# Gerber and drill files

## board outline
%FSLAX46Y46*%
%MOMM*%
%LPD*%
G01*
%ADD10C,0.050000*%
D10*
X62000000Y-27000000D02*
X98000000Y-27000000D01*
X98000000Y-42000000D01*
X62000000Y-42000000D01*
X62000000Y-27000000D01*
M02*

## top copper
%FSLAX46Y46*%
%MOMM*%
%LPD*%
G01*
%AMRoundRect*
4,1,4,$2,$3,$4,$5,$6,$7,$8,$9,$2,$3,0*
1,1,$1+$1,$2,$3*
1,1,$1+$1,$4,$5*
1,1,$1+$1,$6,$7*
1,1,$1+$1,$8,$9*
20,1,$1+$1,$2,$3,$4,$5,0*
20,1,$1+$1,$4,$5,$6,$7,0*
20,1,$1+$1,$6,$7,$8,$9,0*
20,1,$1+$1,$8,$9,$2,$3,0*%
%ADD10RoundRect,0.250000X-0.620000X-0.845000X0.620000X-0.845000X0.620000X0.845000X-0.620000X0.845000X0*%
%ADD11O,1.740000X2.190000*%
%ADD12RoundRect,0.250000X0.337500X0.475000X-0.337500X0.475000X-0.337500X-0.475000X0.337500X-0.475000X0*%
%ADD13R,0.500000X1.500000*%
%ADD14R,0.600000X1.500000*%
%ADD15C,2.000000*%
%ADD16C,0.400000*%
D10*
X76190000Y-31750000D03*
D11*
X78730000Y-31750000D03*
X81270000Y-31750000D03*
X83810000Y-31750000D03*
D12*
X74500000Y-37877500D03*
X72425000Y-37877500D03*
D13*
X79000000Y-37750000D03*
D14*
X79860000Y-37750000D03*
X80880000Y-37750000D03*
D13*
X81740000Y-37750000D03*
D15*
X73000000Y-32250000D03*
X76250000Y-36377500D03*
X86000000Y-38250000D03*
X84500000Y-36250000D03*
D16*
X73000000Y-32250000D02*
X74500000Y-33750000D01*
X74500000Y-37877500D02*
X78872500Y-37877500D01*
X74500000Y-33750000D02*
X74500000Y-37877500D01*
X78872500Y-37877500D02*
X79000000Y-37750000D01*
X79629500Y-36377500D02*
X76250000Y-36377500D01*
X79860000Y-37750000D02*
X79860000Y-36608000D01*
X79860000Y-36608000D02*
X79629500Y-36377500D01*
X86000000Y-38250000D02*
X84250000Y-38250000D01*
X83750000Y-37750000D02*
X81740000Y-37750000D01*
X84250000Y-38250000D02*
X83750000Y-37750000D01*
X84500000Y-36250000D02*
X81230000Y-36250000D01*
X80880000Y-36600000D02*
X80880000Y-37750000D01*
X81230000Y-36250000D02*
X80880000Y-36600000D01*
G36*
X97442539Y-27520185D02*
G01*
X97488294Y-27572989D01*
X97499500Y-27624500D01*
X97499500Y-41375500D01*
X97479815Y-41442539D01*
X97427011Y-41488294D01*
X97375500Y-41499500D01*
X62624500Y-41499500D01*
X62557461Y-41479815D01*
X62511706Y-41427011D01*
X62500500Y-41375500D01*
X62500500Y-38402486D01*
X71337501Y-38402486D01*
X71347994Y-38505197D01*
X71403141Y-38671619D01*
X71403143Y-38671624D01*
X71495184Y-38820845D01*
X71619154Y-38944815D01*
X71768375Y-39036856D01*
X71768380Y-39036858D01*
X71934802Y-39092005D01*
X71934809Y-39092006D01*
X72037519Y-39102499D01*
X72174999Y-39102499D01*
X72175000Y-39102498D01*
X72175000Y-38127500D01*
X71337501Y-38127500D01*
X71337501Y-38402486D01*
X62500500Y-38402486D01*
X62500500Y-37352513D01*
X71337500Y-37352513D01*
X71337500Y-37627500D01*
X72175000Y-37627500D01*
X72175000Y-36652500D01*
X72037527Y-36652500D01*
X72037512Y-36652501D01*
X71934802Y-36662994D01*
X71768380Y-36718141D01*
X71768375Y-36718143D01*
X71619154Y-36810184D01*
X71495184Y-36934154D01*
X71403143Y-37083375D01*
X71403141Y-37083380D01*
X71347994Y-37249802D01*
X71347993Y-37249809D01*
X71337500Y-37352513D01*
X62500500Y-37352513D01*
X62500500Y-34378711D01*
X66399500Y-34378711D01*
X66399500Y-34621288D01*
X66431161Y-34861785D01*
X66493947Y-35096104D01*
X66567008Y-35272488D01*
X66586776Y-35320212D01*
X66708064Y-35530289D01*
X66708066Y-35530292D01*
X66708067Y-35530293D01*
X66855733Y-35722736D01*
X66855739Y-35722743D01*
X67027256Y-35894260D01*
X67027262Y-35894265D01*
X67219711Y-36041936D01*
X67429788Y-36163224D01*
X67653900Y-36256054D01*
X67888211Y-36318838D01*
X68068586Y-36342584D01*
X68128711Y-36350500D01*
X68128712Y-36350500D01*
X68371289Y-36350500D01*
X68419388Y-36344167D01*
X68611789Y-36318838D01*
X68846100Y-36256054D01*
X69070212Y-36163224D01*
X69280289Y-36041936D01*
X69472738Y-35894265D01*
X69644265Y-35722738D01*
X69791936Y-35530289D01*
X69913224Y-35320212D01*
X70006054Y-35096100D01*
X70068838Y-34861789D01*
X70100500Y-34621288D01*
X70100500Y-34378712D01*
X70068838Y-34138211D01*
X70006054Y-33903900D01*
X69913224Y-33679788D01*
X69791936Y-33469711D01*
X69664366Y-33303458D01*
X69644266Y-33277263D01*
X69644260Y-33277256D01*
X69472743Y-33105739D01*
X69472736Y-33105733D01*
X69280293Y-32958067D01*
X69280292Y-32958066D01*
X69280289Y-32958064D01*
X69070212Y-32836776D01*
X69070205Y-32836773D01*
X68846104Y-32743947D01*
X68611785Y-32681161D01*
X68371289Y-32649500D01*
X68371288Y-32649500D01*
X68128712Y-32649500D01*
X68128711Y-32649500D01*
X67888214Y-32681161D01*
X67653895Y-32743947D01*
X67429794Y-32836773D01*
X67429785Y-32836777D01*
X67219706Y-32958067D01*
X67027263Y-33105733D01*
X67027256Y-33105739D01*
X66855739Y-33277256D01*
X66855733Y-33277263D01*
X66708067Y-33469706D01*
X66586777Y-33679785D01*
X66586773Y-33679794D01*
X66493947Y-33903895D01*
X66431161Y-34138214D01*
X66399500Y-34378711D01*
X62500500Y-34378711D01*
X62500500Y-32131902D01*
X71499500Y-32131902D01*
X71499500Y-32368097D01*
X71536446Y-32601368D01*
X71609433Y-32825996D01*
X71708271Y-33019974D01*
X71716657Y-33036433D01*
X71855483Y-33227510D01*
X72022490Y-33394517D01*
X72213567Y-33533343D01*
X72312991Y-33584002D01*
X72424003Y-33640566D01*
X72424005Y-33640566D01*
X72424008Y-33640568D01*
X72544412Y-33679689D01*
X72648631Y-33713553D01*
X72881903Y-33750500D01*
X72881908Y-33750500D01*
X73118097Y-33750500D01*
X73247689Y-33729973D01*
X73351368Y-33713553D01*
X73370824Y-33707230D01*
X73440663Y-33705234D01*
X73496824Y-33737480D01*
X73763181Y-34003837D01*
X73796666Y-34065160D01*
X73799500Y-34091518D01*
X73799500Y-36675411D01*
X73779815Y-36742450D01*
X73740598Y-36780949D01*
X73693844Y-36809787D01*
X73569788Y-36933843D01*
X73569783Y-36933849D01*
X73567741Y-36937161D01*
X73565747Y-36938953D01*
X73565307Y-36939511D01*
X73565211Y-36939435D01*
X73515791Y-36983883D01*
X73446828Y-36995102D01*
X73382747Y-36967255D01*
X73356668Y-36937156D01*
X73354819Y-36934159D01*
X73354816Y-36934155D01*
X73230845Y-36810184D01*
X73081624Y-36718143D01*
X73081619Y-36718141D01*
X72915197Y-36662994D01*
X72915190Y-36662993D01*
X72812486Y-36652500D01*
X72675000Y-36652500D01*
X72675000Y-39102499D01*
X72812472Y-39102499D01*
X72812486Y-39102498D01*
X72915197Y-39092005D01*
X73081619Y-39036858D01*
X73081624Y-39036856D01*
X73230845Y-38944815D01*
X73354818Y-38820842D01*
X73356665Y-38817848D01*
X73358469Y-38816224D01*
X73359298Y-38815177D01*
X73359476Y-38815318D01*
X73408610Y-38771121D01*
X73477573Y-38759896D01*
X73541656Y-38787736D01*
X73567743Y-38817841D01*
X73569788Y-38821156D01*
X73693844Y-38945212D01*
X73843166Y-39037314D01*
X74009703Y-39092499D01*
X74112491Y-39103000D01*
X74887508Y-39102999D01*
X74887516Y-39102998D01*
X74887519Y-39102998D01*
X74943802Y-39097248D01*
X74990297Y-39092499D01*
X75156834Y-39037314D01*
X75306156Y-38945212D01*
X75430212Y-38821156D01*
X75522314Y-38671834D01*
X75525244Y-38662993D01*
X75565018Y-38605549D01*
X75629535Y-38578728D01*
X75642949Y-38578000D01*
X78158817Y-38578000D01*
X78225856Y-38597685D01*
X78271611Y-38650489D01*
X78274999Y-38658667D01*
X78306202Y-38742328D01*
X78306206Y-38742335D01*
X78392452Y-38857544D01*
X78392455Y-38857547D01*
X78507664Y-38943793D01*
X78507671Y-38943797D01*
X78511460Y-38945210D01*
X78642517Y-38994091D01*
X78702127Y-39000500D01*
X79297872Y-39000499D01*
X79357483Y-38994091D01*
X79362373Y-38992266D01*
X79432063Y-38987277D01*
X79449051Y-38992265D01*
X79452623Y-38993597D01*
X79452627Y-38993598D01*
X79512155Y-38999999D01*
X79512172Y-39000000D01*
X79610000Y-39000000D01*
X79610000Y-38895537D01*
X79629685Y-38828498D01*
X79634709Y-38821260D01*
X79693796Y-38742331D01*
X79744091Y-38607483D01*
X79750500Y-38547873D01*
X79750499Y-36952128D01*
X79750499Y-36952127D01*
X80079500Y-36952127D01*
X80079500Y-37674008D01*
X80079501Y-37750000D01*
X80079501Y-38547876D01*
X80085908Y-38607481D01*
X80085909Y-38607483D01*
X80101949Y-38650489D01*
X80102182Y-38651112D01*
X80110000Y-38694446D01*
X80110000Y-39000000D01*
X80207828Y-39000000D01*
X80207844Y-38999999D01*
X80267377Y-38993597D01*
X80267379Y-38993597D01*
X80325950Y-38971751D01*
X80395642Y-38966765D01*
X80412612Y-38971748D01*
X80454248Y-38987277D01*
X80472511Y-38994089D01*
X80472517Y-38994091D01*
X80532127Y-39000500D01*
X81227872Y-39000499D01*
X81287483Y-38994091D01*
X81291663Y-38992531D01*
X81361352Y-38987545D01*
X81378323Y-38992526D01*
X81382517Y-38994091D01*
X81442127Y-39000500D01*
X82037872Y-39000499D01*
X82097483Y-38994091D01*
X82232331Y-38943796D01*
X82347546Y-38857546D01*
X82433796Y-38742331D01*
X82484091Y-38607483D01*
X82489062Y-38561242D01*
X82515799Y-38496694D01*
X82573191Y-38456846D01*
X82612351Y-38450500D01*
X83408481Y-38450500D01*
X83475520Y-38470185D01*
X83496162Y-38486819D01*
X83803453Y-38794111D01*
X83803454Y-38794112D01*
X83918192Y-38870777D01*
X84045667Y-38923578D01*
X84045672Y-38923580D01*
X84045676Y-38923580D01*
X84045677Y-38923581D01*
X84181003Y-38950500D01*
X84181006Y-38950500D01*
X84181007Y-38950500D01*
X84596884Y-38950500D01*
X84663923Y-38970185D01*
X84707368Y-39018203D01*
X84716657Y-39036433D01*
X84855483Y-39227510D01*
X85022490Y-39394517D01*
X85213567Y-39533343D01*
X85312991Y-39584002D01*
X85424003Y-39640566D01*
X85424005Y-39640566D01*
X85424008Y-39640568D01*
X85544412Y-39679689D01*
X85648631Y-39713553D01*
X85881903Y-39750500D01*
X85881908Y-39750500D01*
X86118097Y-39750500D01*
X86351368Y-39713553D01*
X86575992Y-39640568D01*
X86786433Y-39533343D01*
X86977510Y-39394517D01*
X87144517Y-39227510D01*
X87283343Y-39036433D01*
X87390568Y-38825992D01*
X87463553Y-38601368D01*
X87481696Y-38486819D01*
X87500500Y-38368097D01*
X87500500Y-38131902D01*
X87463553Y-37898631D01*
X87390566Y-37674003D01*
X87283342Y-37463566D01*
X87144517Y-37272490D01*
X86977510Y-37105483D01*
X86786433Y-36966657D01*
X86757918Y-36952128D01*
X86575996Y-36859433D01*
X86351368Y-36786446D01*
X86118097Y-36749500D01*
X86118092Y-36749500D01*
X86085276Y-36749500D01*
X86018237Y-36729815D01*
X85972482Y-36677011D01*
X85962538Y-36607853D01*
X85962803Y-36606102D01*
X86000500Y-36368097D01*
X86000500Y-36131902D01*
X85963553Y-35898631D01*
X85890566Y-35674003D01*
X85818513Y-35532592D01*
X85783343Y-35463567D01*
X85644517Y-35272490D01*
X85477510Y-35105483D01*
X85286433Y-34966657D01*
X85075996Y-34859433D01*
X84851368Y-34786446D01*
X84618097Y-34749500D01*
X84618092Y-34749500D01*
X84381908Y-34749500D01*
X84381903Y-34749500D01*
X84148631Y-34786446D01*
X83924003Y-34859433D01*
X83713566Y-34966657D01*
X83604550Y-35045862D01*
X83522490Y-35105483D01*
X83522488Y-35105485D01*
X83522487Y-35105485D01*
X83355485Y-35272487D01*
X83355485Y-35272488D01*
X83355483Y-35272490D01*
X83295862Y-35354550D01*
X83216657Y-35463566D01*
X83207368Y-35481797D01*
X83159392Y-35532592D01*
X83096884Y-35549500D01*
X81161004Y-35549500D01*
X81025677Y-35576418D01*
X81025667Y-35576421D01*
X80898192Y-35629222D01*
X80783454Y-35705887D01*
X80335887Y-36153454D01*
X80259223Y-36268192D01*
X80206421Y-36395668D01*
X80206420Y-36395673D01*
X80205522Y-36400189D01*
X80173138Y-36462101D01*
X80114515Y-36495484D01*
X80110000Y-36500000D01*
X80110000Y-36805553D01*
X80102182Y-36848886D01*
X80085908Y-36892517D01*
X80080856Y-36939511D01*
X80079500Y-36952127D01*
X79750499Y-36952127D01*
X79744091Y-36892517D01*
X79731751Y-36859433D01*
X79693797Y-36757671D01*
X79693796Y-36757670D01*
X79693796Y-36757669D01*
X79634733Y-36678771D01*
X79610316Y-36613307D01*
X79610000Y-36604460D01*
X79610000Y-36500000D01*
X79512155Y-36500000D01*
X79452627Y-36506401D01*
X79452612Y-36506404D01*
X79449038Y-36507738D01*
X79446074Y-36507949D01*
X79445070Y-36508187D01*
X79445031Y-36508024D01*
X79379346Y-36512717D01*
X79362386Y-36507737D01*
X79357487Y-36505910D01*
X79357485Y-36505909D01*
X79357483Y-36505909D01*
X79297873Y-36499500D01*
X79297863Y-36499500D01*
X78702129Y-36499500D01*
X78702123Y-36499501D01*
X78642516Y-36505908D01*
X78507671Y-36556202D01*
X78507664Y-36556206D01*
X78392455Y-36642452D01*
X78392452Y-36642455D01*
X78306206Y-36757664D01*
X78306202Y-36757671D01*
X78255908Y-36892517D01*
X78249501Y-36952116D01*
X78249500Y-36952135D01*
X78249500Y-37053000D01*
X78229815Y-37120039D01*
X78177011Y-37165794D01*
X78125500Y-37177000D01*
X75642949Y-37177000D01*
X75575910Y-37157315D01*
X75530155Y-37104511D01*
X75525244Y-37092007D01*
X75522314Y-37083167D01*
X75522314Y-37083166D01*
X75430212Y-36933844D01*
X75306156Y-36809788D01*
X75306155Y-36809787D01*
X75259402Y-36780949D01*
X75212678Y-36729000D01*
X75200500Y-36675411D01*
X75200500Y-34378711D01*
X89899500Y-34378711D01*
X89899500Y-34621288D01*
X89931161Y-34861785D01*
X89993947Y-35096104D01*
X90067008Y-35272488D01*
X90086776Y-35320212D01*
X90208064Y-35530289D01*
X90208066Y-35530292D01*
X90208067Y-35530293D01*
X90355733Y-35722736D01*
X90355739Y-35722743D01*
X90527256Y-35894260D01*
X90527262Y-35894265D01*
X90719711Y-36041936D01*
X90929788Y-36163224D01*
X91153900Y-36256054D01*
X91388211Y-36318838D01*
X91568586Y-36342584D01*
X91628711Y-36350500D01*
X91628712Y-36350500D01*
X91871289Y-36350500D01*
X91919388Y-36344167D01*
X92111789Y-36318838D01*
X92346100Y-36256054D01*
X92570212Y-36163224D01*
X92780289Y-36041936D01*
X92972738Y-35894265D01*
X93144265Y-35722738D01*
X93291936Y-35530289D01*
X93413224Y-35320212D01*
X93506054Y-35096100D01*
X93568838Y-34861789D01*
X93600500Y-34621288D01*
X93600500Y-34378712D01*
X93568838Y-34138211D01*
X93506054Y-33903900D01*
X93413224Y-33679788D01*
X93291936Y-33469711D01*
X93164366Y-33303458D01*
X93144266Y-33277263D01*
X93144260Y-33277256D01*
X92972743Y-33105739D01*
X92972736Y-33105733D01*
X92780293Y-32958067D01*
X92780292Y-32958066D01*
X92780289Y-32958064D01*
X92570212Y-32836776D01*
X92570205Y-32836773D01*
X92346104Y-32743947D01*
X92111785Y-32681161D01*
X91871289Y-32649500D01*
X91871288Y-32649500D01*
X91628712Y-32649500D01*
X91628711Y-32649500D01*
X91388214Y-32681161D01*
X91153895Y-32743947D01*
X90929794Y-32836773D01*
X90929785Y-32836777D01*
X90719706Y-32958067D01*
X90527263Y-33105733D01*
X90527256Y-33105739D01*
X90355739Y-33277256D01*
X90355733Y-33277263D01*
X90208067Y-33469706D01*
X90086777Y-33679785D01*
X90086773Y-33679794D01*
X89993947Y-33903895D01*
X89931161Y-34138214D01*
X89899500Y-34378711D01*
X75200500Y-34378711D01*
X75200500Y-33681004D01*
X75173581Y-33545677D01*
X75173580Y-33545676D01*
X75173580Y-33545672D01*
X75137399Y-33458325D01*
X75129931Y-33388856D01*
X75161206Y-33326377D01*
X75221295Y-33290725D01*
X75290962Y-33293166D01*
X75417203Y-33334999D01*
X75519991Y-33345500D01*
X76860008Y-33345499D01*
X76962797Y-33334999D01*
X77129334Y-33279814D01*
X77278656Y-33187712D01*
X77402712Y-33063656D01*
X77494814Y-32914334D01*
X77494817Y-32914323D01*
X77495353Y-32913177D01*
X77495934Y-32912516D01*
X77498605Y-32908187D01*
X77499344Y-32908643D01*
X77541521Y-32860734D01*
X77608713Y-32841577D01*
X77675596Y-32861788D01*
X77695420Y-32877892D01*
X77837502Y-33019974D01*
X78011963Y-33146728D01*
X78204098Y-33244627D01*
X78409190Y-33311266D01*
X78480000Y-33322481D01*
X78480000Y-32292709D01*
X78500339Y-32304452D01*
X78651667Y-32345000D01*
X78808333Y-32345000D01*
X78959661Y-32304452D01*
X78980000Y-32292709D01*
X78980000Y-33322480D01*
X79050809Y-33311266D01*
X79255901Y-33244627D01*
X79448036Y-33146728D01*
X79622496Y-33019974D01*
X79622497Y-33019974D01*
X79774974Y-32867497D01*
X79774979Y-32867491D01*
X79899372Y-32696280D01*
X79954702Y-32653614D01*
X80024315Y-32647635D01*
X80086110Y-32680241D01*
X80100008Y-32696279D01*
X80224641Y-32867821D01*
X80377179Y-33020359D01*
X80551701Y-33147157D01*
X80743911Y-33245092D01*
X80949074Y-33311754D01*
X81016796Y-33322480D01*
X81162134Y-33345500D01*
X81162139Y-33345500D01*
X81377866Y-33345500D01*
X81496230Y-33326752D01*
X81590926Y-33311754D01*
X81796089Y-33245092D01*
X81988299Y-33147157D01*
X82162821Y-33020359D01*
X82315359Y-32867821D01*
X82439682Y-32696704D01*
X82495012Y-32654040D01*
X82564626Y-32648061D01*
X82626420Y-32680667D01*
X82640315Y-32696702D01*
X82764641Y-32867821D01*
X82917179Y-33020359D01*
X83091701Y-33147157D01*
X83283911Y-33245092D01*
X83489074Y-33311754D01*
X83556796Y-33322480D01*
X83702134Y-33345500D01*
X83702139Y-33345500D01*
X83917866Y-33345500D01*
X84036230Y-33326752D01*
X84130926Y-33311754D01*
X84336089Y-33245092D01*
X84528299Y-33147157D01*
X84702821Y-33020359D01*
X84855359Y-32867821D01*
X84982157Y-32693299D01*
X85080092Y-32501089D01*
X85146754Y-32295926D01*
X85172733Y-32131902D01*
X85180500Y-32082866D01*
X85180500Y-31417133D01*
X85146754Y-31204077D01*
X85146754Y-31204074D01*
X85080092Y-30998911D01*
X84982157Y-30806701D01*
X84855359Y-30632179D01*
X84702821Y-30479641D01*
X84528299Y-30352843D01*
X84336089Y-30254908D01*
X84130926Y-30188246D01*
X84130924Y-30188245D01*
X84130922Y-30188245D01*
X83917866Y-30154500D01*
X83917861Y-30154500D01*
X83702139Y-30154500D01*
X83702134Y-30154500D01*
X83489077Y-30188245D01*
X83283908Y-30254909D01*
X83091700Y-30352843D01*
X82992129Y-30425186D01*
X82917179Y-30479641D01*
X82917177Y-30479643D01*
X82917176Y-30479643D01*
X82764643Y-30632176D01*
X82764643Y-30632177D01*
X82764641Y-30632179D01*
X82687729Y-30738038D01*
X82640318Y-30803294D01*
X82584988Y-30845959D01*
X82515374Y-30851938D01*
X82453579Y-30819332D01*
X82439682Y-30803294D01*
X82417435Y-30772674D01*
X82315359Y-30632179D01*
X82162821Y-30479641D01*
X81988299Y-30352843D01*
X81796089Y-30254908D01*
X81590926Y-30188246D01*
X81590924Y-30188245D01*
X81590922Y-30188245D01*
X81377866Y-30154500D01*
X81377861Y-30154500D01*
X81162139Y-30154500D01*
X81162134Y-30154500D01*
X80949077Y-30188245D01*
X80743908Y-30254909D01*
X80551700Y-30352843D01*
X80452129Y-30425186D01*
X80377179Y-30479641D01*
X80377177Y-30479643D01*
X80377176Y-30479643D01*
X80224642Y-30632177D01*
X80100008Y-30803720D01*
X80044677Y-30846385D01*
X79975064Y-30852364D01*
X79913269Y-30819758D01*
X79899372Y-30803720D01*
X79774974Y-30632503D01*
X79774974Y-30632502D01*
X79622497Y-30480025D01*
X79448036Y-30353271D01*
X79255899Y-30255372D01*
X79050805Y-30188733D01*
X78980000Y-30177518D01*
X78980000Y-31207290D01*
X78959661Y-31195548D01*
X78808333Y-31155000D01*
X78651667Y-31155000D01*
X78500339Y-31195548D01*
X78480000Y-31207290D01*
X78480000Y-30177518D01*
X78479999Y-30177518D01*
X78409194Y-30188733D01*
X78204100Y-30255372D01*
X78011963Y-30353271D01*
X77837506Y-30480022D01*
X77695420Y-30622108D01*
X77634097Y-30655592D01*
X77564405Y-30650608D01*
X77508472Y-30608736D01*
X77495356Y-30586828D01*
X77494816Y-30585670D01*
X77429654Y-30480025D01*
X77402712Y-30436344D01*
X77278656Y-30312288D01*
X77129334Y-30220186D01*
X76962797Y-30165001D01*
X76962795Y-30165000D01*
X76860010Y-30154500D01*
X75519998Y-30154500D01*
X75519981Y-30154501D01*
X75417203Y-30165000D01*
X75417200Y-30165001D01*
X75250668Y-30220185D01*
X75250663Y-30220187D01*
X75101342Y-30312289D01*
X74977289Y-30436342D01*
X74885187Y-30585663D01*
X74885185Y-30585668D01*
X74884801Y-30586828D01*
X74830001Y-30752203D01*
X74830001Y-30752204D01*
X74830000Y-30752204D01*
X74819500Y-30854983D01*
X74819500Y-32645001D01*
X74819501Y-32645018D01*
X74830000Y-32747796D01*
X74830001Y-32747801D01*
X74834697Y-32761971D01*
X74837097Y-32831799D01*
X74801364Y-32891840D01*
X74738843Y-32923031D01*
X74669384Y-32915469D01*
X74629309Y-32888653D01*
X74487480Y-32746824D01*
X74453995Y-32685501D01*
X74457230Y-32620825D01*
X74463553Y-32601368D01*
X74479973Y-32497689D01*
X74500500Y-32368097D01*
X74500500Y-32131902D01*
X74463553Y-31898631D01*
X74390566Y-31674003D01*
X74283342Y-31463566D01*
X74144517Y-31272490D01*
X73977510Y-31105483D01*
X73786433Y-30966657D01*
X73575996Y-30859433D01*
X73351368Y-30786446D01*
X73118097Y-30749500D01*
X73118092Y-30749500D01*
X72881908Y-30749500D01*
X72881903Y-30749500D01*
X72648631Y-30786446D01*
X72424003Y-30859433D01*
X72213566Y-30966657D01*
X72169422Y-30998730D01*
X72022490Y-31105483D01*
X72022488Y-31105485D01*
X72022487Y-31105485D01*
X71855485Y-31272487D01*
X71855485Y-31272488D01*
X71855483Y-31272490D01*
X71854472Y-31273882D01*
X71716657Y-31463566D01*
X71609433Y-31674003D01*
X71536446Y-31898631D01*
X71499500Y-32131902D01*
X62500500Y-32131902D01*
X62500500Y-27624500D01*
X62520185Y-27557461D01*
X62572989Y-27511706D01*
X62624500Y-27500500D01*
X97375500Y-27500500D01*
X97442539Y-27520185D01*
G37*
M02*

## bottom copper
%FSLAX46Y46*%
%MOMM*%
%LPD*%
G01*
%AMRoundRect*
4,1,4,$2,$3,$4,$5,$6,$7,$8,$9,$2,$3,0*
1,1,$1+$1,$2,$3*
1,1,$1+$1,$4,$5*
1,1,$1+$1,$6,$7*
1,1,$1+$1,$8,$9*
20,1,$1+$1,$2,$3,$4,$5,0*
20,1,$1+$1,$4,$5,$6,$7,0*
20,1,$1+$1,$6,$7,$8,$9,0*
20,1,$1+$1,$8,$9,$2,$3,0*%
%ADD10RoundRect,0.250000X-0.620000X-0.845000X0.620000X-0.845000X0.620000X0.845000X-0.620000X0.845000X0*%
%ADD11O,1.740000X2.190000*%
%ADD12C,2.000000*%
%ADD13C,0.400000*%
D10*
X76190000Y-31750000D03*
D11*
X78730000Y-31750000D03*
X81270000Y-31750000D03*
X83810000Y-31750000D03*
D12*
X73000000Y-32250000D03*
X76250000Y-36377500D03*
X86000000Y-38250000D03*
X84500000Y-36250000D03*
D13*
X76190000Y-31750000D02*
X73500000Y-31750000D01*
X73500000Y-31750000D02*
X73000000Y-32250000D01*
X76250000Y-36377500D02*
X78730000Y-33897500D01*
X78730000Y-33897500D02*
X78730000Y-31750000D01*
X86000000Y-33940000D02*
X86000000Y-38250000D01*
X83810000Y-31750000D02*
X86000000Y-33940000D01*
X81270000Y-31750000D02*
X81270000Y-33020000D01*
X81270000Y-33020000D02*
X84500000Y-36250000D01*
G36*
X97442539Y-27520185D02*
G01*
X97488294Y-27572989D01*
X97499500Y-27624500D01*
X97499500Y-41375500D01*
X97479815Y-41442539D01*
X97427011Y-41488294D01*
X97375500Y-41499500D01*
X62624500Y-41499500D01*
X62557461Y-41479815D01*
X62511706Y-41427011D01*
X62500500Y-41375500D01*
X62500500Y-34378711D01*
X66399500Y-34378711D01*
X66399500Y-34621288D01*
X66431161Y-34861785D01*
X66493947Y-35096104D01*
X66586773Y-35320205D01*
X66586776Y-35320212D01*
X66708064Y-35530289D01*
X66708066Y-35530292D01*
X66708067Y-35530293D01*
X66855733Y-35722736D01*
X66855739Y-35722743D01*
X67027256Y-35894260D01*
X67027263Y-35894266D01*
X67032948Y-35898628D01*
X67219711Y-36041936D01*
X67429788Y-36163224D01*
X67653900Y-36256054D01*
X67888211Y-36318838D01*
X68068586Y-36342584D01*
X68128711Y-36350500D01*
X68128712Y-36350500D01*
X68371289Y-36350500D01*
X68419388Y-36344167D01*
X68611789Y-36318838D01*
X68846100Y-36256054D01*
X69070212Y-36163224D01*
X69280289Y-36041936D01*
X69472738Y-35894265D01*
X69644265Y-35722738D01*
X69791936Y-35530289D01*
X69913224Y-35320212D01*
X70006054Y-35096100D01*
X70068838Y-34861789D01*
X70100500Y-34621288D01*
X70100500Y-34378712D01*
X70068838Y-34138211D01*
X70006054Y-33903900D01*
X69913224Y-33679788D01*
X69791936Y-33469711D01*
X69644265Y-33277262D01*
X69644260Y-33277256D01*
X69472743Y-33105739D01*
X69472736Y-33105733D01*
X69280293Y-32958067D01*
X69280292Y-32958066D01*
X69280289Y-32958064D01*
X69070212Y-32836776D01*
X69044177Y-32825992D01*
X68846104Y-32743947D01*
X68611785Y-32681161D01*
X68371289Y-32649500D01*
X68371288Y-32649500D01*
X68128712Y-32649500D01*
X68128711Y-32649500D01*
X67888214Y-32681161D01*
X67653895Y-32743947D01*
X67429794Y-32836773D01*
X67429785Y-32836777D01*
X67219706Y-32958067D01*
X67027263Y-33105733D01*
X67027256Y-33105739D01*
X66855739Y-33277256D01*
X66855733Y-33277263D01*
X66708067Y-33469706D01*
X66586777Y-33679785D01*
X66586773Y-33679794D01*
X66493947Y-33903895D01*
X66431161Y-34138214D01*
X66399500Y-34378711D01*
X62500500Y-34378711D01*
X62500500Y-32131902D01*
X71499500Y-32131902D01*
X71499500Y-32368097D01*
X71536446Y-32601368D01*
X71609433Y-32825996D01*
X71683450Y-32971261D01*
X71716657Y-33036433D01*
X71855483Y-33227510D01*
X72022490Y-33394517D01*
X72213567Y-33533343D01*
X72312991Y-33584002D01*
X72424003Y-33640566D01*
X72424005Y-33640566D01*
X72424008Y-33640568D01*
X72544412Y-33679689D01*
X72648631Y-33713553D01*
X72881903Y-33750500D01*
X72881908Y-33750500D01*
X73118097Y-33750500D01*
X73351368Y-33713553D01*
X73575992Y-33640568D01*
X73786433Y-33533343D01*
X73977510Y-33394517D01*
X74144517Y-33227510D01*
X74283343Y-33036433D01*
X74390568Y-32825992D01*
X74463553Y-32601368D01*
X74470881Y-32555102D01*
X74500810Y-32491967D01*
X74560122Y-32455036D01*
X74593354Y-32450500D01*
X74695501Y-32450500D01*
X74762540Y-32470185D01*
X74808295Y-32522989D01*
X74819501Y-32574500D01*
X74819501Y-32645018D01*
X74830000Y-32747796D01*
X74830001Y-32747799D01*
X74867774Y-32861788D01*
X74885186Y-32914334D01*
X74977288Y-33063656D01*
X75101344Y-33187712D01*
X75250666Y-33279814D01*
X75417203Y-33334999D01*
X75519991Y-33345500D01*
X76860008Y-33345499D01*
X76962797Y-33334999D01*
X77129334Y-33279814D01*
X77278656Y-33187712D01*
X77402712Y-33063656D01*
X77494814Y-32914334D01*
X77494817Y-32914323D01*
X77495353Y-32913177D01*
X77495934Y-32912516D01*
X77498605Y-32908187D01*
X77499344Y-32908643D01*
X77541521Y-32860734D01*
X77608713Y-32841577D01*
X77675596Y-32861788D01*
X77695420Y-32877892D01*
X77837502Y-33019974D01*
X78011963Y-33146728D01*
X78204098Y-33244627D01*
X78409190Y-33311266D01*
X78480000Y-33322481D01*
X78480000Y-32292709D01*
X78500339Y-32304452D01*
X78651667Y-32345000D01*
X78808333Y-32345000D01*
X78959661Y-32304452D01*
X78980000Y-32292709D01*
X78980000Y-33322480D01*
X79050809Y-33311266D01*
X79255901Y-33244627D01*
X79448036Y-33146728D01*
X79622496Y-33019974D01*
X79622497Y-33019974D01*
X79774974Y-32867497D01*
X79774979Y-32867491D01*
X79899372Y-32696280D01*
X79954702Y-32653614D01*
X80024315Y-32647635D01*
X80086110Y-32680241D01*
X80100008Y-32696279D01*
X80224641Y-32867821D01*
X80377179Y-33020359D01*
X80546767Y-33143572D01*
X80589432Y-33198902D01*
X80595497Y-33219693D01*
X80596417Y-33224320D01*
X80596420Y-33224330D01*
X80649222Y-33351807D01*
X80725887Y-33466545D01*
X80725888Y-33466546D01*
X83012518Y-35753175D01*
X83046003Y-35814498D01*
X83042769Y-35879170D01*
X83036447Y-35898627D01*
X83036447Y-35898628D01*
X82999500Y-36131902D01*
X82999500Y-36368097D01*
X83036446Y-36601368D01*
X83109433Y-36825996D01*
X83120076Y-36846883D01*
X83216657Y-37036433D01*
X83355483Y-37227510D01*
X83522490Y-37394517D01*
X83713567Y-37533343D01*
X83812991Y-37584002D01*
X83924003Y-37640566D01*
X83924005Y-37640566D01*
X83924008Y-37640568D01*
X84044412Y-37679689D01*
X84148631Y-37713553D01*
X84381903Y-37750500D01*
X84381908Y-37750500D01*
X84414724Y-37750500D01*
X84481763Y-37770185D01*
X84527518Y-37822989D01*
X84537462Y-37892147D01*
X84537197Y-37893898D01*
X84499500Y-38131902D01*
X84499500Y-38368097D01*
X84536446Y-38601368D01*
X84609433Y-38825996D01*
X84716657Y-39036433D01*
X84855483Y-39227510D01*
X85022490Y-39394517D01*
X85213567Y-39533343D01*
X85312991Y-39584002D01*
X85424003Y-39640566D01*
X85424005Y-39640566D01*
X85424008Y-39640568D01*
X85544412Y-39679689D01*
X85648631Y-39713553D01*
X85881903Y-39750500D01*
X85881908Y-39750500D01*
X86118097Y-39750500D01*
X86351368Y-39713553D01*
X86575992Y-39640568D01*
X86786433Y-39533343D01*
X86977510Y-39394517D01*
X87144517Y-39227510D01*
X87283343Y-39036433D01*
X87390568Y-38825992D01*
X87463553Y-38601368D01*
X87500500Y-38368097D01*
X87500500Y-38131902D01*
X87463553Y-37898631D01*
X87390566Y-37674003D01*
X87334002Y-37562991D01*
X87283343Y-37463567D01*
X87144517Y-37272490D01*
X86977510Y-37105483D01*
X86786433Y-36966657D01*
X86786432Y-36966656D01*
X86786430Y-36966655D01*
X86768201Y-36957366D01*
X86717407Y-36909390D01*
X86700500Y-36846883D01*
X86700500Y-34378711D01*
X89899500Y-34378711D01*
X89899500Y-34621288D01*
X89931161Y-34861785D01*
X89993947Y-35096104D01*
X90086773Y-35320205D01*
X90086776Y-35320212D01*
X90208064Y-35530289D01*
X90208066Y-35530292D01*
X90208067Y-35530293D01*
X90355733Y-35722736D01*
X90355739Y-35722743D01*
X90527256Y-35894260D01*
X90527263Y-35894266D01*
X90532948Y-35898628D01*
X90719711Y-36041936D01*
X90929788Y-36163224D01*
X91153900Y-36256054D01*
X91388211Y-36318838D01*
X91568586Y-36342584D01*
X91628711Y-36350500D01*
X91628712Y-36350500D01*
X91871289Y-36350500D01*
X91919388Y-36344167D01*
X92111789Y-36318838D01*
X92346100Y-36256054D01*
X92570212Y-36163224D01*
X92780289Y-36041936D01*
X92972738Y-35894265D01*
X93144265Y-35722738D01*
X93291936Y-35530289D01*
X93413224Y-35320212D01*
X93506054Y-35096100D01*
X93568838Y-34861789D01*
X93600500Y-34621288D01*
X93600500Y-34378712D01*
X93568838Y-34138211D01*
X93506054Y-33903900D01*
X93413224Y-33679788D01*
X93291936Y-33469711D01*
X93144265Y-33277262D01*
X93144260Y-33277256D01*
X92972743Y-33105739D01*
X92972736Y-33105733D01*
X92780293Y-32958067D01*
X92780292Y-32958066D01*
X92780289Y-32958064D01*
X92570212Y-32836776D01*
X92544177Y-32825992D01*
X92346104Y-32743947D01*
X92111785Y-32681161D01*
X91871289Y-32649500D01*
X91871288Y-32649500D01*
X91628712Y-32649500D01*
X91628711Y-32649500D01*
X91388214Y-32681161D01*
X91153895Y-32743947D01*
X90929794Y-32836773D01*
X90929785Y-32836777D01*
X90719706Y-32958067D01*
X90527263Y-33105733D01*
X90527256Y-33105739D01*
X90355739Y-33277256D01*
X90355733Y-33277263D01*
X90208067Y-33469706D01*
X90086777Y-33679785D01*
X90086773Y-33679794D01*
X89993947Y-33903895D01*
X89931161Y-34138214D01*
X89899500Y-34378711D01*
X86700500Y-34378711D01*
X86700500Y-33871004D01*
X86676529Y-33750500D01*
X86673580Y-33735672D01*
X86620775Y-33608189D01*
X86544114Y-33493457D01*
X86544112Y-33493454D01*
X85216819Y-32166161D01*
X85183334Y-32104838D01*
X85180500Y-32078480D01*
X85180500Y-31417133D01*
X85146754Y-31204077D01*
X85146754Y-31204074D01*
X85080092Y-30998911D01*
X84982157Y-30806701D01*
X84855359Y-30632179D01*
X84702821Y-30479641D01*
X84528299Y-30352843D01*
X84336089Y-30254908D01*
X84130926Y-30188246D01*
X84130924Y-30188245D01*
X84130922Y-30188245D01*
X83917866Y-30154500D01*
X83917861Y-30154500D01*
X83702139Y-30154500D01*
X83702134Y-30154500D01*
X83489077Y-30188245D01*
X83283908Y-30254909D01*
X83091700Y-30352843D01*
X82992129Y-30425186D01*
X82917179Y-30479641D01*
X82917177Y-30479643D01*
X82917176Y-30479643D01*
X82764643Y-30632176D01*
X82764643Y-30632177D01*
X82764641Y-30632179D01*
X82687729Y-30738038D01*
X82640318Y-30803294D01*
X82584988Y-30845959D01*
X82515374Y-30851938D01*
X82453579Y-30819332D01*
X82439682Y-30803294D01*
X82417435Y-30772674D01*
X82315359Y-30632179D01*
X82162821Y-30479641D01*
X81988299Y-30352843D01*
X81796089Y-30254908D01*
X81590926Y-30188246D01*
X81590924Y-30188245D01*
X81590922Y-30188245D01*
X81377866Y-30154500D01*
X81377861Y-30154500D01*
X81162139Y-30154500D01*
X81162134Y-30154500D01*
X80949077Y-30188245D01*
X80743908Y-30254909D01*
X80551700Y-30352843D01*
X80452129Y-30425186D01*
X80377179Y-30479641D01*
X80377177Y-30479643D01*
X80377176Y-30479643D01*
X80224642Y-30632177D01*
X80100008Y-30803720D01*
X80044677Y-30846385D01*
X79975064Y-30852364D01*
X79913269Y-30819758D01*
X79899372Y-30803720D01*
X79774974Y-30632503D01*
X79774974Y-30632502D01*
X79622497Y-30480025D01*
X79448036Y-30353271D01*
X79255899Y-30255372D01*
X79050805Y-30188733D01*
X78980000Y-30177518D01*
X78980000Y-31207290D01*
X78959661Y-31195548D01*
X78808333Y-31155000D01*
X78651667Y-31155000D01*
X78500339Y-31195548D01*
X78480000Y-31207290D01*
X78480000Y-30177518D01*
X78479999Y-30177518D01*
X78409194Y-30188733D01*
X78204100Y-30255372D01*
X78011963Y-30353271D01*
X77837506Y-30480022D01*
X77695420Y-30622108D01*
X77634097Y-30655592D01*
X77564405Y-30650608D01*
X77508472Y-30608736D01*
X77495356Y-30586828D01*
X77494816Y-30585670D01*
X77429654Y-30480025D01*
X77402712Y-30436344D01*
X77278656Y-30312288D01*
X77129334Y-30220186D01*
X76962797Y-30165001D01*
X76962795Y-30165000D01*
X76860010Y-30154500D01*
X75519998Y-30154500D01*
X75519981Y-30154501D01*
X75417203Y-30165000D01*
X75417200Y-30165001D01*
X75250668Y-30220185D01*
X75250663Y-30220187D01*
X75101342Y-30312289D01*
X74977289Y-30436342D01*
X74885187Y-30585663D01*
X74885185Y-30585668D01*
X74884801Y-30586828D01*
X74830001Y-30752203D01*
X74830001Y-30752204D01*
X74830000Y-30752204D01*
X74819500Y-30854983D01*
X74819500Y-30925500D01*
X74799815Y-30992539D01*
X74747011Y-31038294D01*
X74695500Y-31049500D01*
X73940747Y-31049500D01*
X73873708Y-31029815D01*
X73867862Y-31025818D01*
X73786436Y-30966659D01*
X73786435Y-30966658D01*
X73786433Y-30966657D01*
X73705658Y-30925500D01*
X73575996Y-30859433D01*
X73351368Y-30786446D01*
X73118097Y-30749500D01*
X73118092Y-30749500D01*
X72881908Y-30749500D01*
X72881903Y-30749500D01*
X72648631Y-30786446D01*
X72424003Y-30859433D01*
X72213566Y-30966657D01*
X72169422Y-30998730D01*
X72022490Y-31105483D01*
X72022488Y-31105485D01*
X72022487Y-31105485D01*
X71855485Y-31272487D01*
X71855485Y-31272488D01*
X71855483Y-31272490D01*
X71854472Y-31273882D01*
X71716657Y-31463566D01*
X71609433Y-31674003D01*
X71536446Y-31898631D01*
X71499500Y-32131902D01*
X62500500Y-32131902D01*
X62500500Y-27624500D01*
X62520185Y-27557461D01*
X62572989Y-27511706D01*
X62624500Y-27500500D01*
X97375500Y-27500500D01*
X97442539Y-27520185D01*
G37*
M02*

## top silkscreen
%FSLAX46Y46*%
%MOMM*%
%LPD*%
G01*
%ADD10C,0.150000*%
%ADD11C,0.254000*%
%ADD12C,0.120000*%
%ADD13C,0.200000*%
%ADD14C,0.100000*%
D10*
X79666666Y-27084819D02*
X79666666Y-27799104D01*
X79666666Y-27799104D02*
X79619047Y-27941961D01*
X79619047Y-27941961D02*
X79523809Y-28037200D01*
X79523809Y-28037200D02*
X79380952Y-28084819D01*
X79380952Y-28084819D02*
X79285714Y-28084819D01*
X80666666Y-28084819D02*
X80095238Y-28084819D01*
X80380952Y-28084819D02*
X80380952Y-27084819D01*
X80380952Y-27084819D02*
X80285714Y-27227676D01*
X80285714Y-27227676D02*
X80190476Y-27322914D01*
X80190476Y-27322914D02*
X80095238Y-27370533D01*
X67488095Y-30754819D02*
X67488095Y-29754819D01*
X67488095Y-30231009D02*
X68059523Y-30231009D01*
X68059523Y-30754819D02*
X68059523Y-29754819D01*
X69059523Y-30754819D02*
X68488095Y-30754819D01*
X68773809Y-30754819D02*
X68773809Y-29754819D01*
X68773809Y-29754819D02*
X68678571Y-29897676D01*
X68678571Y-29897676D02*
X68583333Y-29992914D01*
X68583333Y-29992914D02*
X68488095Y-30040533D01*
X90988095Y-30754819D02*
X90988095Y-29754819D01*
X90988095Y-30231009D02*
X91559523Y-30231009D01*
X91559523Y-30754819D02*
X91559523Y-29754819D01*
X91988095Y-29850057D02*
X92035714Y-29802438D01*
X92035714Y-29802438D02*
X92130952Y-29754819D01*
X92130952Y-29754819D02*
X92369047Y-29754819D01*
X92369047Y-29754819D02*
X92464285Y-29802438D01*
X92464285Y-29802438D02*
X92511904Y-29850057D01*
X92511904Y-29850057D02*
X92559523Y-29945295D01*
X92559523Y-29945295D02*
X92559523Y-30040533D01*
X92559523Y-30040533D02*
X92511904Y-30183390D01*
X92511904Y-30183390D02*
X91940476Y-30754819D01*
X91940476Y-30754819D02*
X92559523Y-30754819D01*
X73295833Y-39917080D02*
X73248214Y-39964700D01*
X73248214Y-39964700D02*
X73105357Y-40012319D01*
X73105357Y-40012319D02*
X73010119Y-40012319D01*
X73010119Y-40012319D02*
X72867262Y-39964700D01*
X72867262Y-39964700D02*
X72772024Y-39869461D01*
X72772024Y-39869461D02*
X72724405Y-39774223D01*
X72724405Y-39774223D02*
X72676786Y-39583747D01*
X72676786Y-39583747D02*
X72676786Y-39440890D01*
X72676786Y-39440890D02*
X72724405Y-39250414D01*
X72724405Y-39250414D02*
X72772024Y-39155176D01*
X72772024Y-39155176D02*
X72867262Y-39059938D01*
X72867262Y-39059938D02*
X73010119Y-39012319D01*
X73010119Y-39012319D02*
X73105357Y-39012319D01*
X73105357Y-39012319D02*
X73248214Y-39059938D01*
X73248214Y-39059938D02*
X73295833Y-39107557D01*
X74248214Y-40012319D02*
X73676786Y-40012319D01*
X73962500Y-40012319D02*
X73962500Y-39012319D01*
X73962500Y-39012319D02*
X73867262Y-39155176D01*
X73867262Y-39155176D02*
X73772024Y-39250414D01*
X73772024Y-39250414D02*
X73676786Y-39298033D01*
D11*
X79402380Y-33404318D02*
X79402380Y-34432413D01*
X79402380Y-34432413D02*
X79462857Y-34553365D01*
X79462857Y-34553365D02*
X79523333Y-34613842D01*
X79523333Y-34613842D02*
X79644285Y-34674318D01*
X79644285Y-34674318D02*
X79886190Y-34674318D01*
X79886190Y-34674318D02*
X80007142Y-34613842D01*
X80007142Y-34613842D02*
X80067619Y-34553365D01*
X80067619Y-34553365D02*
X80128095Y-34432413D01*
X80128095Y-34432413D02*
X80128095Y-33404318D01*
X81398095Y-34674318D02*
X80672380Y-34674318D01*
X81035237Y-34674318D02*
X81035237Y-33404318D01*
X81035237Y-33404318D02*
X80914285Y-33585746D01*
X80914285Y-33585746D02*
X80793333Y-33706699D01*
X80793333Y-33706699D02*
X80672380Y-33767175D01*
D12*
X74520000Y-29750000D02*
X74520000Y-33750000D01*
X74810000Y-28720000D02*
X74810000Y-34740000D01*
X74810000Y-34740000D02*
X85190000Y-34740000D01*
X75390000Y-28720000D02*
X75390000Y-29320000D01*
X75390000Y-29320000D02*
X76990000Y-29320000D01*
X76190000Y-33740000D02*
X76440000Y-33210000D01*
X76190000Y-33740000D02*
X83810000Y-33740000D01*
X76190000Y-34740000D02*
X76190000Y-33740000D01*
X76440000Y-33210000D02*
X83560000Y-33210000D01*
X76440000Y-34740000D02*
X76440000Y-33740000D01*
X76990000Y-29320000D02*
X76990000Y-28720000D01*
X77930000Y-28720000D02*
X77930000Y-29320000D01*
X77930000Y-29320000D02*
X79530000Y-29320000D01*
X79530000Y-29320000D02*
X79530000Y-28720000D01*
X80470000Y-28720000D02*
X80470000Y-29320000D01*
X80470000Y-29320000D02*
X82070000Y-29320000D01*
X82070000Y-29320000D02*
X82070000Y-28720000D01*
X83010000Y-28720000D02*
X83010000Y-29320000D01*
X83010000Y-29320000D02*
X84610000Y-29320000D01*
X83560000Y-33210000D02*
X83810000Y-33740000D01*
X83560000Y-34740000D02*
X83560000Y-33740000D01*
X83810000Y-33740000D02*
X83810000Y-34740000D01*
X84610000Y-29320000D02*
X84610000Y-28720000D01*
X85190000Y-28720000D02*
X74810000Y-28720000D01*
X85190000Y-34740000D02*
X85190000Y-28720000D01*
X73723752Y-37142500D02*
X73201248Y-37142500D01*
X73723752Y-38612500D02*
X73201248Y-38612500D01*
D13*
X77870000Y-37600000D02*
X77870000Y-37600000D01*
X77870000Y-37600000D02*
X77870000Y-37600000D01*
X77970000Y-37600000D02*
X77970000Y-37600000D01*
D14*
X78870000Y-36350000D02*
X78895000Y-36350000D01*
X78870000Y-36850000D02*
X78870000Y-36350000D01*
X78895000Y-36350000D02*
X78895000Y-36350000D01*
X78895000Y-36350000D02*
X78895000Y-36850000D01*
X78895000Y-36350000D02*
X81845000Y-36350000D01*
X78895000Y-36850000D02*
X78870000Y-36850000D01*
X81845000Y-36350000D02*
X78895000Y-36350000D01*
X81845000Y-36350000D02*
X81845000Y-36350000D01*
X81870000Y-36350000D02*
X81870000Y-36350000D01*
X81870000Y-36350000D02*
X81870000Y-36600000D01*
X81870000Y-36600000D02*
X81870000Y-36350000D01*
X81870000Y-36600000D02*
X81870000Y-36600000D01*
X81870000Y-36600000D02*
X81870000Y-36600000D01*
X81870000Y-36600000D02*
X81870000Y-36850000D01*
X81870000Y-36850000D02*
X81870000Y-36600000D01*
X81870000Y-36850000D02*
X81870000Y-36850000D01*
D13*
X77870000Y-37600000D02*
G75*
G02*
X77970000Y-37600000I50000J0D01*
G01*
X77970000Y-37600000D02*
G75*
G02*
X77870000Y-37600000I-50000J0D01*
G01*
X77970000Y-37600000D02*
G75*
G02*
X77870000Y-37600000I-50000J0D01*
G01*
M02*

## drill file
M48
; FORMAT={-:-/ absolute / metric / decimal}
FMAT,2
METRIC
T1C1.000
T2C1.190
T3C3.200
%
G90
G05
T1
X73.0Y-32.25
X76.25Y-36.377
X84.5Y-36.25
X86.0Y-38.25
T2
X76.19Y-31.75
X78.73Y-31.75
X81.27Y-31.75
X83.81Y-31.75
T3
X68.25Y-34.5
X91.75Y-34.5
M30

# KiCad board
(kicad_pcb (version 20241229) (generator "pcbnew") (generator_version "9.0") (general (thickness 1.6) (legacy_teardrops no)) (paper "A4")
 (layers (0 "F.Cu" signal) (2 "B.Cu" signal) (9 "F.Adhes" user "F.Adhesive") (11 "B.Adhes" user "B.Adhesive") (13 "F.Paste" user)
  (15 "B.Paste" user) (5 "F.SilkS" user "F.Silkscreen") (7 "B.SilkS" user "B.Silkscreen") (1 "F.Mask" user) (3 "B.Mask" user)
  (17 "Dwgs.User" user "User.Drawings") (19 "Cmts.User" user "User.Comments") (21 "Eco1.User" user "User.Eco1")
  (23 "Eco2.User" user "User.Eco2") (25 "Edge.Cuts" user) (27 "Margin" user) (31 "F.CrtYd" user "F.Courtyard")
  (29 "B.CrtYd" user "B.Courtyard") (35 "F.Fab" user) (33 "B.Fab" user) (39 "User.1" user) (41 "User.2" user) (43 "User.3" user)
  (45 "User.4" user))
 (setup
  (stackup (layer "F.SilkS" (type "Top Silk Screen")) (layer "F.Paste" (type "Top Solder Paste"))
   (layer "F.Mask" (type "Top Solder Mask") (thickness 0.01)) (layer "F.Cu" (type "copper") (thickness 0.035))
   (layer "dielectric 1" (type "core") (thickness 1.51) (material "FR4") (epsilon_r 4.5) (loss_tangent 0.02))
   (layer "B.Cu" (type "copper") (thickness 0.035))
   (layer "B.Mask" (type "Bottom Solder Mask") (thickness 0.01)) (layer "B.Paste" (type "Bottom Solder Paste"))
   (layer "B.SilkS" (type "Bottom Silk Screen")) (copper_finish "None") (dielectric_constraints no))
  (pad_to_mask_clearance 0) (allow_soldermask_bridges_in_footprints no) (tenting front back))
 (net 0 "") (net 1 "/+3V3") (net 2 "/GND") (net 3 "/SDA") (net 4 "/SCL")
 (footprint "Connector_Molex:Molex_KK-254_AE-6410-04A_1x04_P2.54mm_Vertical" (layer "F.Cu") (at 76.19 31.75)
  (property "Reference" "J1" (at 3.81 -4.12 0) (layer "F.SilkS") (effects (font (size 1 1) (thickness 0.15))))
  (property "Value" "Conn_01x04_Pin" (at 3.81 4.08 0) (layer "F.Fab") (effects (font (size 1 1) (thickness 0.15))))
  (fp_line (start -1.67 -2) (end -1.67 2) (stroke (width 0.12) (type solid)) (layer "F.SilkS"))
  (fp_line (start -1.38 -3.03) (end -1.38 2.99) (stroke (width 0.12) (type solid)) (layer "F.SilkS"))
  (fp_line (start -1.38 2.99) (end 9 2.99) (stroke (width 0.12) (type solid)) (layer "F.SilkS"))
  (fp_line (start -0.8 -3.03) (end -0.8 -2.43) (stroke (width 0.12) (type solid)) (layer "F.SilkS"))
  (fp_line (start -0.8 -2.43) (end 0.8 -2.43) (stroke (width 0.12) (type solid)) (layer "F.SilkS"))
  (fp_line (start 0 1.99) (end 0.25 1.46) (stroke (width 0.12) (type solid)) (layer "F.SilkS"))
  (fp_line (start 0 1.99) (end 7.62 1.99) (stroke (width 0.12) (type solid)) (layer "F.SilkS"))
  (fp_line (start 0 2.99) (end 0 1.99) (stroke (width 0.12) (type solid)) (layer "F.SilkS"))
  (fp_line (start 0.25 1.46) (end 7.37 1.46) (stroke (width 0.12) (type solid)) (layer "F.SilkS"))
  (fp_line (start 0.25 2.99) (end 0.25 1.99) (stroke (width 0.12) (type solid)) (layer "F.SilkS"))
  (fp_line (start 0.8 -2.43) (end 0.8 -3.03) (stroke (width 0.12) (type solid)) (layer "F.SilkS"))
  (fp_line (start 1.74 -3.03) (end 1.74 -2.43) (stroke (width 0.12) (type solid)) (layer "F.SilkS"))
  (fp_line (start 1.74 -2.43) (end 3.34 -2.43) (stroke (width 0.12) (type solid)) (layer "F.SilkS"))
  (fp_line (start 3.34 -2.43) (end 3.34 -3.03) (stroke (width 0.12) (type solid)) (layer "F.SilkS"))
  (fp_line (start 4.28 -3.03) (end 4.28 -2.43) (stroke (width 0.12) (type solid)) (layer "F.SilkS"))
  (fp_line (start 4.28 -2.43) (end 5.88 -2.43) (stroke (width 0.12) (type solid)) (layer "F.SilkS"))
  (fp_line (start 5.88 -2.43) (end 5.88 -3.03) (stroke (width 0.12) (type solid)) (layer "F.SilkS"))
  (fp_line (start 6.82 -3.03) (end 6.82 -2.43) (stroke (width 0.12) (type solid)) (layer "F.SilkS"))
  (fp_line (start 6.82 -2.43) (end 8.42 -2.43) (stroke (width 0.12) (type solid)) (layer "F.SilkS"))
  (fp_line (start 7.37 1.46) (end 7.62 1.99) (stroke (width 0.12) (type solid)) (layer "F.SilkS"))
  (fp_line (start 7.37 2.99) (end 7.37 1.99) (stroke (width 0.12) (type solid)) (layer "F.SilkS"))
  (fp_line (start 7.62 1.99) (end 7.62 2.99) (stroke (width 0.12) (type solid)) (layer "F.SilkS"))
  (fp_line (start 8.42 -2.43) (end 8.42 -3.03) (stroke (width 0.12) (type solid)) (layer "F.SilkS"))
  (fp_line (start 9 -3.03) (end -1.38 -3.03) (stroke (width 0.12) (type solid)) (layer "F.SilkS"))
  (fp_line (start 9 2.99) (end 9 -3.03) (stroke (width 0.12) (type solid)) (layer "F.SilkS"))
  (pad "1" thru_hole roundrect (at 0 0) (size 1.74 2.19) (drill 1.19) (layers "*.Cu" "*.Mask") (remove_unused_layers no)
   (roundrect_rratio 0.143678) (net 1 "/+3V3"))
  (pad "2" thru_hole oval (at 2.54 0) (size 1.74 2.19) (drill 1.19) (layers "*.Cu" "*.Mask") (remove_unused_layers no) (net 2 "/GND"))
  (pad "3" thru_hole oval (at 5.08 0) (size 1.74 2.19) (drill 1.19) (layers "*.Cu" "*.Mask") (remove_unused_layers no) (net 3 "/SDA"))
  (pad "4" thru_hole oval (at 7.62 0) (size 1.74 2.19) (drill 1.19) (layers "*.Cu" "*.Mask") (remove_unused_layers no) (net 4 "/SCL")))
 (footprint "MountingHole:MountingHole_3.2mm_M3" (layer "F.Cu") (at 68.25 34.5)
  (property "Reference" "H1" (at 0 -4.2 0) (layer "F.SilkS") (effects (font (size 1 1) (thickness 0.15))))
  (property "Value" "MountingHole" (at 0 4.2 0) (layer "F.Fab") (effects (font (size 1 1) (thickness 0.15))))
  (pad "" np_thru_hole circle (at 0 0) (size 3.2 3.2) (drill 3.2) (layers "*.Cu" "*.Mask")))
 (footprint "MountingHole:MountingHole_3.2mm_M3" (layer "F.Cu") (at 91.75 34.5)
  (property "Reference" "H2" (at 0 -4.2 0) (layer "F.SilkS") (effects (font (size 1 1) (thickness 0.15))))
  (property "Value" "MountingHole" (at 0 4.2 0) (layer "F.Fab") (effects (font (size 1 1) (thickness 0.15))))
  (pad "" np_thru_hole circle (at 0 0) (size 3.2 3.2) (drill 3.2) (layers "*.Cu" "*.Mask")))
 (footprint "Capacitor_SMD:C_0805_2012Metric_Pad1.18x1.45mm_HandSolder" (layer "F.Cu") (at 73.4625 37.8775 180)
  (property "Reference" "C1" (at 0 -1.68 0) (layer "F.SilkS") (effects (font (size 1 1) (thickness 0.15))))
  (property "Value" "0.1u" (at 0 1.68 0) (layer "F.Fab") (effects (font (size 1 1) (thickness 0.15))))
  (fp_line (start -0.261252 0.735) (end 0.261252 0.735) (stroke (width 0.12) (type solid)) (layer "F.SilkS"))
  (fp_line (start -0.261252 -0.735) (end 0.261252 -0.735) (stroke (width 0.12) (type solid)) (layer "F.SilkS"))
  (pad "1" smd roundrect (at -1.0375 0 180) (size 1.175 1.45) (layers "F.Cu" "F.Mask" "F.Paste") (roundrect_rratio 0.212766) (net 1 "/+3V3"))
  (pad "2" smd roundrect (at 1.0375 0 180) (size 1.175 1.45) (layers "F.Cu" "F.Mask" "F.Paste") (roundrect_rratio 0.212766) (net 2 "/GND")))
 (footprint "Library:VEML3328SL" (layer "F.Cu") (at 80.37 37.1)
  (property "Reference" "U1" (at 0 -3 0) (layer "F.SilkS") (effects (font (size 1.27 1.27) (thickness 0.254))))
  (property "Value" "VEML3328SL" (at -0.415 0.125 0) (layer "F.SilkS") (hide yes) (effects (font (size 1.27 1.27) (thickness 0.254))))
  (fp_line (start -2.5 0.5) (end -2.5 0.5) (stroke (width 0.2) (type solid)) (layer "F.SilkS"))
  (fp_line (start -2.5 0.5) (end -2.5 0.5) (stroke (width 0.2) (type solid)) (layer "F.SilkS"))
  (fp_line (start -2.4 0.5) (end -2.4 0.5) (stroke (width 0.2) (type solid)) (layer "F.SilkS"))
  (fp_line (start -1.5 -0.75) (end -1.475 -0.75) (stroke (width 0.1) (type solid)) (layer "F.SilkS"))
  (fp_line (start -1.5 -0.25) (end -1.5 -0.75) (stroke (width 0.1) (type solid)) (layer "F.SilkS"))
  (fp_line (start -1.475 -0.75) (end -1.475 -0.75) (stroke (width 0.1) (type solid)) (layer "F.SilkS"))
  (fp_line (start -1.475 -0.75) (end -1.475 -0.25) (stroke (width 0.1) (type solid)) (layer "F.SilkS"))
  (fp_line (start -1.475 -0.75) (end 1.475 -0.75) (stroke (width 0.1) (type solid)) (layer "F.SilkS"))
  (fp_line (start -1.475 -0.25) (end -1.5 -0.25) (stroke (width 0.1) (type solid)) (layer "F.SilkS"))
  (fp_line (start 1.475 -0.75) (end -1.475 -0.75) (stroke (width 0.1) (type solid)) (layer "F.SilkS"))
  (fp_line (start 1.475 -0.75) (end 1.475 -0.75) (stroke (width 0.1) (type solid)) (layer "F.SilkS"))
  (fp_line (start 1.5 -0.75) (end 1.5 -0.75) (stroke (width 0.1) (type solid)) (layer "F.SilkS"))
  (fp_line (start 1.5 -0.75) (end 1.5 -0.5) (stroke (width 0.1) (type solid)) (layer "F.SilkS"))
  (fp_line (start 1.5 -0.5) (end 1.5 -0.75) (stroke (width 0.1) (type solid)) (layer "F.SilkS"))
  (fp_line (start 1.5 -0.5) (end 1.5 -0.5) (stroke (width 0.1) (type solid)) (layer "F.SilkS"))
  (fp_line (start 1.5 -0.5) (end 1.5 -0.5) (stroke (width 0.1) (type solid)) (layer "F.SilkS"))
  (fp_line (start 1.5 -0.5) (end 1.5 -0.25) (stroke (width 0.1) (type solid)) (layer "F.SilkS"))
  (fp_line (start 1.5 -0.25) (end 1.5 -0.5) (stroke (width 0.1) (type solid)) (layer "F.SilkS"))
  (fp_line (start 1.5 -0.25) (end 1.5 -0.25) (stroke (width 0.1) (type solid)) (layer "F.SilkS"))
  (fp_arc (start -2.5 0.5) (mid -2.45 0.45) (end -2.4 0.5) (stroke (width 0.2) (type solid)) (layer "F.SilkS"))
  (fp_arc (start -2.4 0.5) (mid -2.45 0.55) (end -2.5 0.5) (stroke (width 0.2) (type solid)) (layer "F.SilkS"))
  (fp_arc (start -2.4 0.5) (mid -2.45 0.55) (end -2.5 0.5) (stroke (width 0.2) (type solid)) (layer "F.SilkS"))
  (pad "1" smd rect (at -1.37 0.65) (size 0.5 1.5) (layers "F.Cu" "F.Mask" "F.Paste") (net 1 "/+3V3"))
  (pad "2" smd rect (at -0.51 0.65 90) (size 1.5 0.6) (layers "F.Cu" "F.Mask" "F.Paste") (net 2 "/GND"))
  (pad "3" smd rect (at 0.51 0.65 90) (size 1.5 0.6) (layers "F.Cu" "F.Mask" "F.Paste") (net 3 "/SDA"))
  (pad "4" smd rect (at 1.37 0.65) (size 0.5 1.5) (layers "F.Cu" "F.Mask" "F.Paste") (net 4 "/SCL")))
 (gr_rect (start 62 27) (end 98 42) (stroke (width 0.05) (type solid)) (fill no) (layer "Edge.Cuts"))
 (segment (start 73 32.25) (end 74.5 33.75) (width 0.4) (layer "F.Cu") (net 1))
 (segment (start 74.5 37.8775) (end 78.8725 37.8775) (width 0.4) (layer "F.Cu") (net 1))
 (segment (start 74.5 33.75) (end 74.5 37.8775) (width 0.4) (layer "F.Cu") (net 1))
 (segment (start 78.8725 37.8775) (end 79 37.75) (width 0.4) (layer "F.Cu") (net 1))
 (via (at 73 32.25) (size 2) (drill 1) (layers "F.Cu" "B.Cu") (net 1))
 (segment (start 76.19 31.75) (end 73.5 31.75) (width 0.4) (layer "B.Cu") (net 1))
 (segment (start 73.5 31.75) (end 73 32.25) (width 0.4) (layer "B.Cu") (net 1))
 (segment (start 79.6295 36.3775) (end 76.25 36.3775) (width 0.4) (layer "F.Cu") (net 2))
 (segment (start 79.86 37.75) (end 79.86 36.608) (width 0.4) (layer "F.Cu") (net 2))
 (segment (start 79.86 36.608) (end 79.6295 36.3775) (width 0.4) (layer "F.Cu") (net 2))
 (via (at 76.25 36.3775) (size 2) (drill 1) (layers "F.Cu" "B.Cu") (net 2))
 (segment (start 76.25 36.3775) (end 78.73 33.8975) (width 0.4) (layer "B.Cu") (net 2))
 (segment (start 78.73 33.8975) (end 78.73 31.75) (width 0.4) (layer "B.Cu") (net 2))
 (segment (start 86 38.25) (end 84.25 38.25) (width 0.4) (layer "F.Cu") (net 4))
 (segment (start 83.75 37.75) (end 81.74 37.75) (width 0.4) (layer "F.Cu") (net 4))
 (segment (start 84.25 38.25) (end 83.75 37.75) (width 0.4) (layer "F.Cu") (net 4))
 (via (at 86 38.25) (size 2) (drill 1) (layers "F.Cu" "B.Cu") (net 4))
 (segment (start 86 33.94) (end 86 38.25) (width 0.4) (layer "B.Cu") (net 4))
 (segment (start 83.81 31.75) (end 86 33.94) (width 0.4) (layer "B.Cu") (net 4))
 (segment (start 84.5 36.25) (end 81.23 36.25) (width 0.4) (layer "F.Cu") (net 3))
 (segment (start 80.88 36.6) (end 80.88 37.75) (width 0.4) (layer "F.Cu") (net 3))
 (segment (start 81.23 36.25) (end 80.88 36.6) (width 0.4) (layer "F.Cu") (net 3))
 (via (at 84.5 36.25) (size 2) (drill 1) (layers "F.Cu" "B.Cu") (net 3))
 (segment (start 81.27 31.75) (end 81.27 33.02) (width 0.4) (layer "B.Cu") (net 3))
 (segment (start 81.27 33.02) (end 84.5 36.25) (width 0.4) (layer "B.Cu") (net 3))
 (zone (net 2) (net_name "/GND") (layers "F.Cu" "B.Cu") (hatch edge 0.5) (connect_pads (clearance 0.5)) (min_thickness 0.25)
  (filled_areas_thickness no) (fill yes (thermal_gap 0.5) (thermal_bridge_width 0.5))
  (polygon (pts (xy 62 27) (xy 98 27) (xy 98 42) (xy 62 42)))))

